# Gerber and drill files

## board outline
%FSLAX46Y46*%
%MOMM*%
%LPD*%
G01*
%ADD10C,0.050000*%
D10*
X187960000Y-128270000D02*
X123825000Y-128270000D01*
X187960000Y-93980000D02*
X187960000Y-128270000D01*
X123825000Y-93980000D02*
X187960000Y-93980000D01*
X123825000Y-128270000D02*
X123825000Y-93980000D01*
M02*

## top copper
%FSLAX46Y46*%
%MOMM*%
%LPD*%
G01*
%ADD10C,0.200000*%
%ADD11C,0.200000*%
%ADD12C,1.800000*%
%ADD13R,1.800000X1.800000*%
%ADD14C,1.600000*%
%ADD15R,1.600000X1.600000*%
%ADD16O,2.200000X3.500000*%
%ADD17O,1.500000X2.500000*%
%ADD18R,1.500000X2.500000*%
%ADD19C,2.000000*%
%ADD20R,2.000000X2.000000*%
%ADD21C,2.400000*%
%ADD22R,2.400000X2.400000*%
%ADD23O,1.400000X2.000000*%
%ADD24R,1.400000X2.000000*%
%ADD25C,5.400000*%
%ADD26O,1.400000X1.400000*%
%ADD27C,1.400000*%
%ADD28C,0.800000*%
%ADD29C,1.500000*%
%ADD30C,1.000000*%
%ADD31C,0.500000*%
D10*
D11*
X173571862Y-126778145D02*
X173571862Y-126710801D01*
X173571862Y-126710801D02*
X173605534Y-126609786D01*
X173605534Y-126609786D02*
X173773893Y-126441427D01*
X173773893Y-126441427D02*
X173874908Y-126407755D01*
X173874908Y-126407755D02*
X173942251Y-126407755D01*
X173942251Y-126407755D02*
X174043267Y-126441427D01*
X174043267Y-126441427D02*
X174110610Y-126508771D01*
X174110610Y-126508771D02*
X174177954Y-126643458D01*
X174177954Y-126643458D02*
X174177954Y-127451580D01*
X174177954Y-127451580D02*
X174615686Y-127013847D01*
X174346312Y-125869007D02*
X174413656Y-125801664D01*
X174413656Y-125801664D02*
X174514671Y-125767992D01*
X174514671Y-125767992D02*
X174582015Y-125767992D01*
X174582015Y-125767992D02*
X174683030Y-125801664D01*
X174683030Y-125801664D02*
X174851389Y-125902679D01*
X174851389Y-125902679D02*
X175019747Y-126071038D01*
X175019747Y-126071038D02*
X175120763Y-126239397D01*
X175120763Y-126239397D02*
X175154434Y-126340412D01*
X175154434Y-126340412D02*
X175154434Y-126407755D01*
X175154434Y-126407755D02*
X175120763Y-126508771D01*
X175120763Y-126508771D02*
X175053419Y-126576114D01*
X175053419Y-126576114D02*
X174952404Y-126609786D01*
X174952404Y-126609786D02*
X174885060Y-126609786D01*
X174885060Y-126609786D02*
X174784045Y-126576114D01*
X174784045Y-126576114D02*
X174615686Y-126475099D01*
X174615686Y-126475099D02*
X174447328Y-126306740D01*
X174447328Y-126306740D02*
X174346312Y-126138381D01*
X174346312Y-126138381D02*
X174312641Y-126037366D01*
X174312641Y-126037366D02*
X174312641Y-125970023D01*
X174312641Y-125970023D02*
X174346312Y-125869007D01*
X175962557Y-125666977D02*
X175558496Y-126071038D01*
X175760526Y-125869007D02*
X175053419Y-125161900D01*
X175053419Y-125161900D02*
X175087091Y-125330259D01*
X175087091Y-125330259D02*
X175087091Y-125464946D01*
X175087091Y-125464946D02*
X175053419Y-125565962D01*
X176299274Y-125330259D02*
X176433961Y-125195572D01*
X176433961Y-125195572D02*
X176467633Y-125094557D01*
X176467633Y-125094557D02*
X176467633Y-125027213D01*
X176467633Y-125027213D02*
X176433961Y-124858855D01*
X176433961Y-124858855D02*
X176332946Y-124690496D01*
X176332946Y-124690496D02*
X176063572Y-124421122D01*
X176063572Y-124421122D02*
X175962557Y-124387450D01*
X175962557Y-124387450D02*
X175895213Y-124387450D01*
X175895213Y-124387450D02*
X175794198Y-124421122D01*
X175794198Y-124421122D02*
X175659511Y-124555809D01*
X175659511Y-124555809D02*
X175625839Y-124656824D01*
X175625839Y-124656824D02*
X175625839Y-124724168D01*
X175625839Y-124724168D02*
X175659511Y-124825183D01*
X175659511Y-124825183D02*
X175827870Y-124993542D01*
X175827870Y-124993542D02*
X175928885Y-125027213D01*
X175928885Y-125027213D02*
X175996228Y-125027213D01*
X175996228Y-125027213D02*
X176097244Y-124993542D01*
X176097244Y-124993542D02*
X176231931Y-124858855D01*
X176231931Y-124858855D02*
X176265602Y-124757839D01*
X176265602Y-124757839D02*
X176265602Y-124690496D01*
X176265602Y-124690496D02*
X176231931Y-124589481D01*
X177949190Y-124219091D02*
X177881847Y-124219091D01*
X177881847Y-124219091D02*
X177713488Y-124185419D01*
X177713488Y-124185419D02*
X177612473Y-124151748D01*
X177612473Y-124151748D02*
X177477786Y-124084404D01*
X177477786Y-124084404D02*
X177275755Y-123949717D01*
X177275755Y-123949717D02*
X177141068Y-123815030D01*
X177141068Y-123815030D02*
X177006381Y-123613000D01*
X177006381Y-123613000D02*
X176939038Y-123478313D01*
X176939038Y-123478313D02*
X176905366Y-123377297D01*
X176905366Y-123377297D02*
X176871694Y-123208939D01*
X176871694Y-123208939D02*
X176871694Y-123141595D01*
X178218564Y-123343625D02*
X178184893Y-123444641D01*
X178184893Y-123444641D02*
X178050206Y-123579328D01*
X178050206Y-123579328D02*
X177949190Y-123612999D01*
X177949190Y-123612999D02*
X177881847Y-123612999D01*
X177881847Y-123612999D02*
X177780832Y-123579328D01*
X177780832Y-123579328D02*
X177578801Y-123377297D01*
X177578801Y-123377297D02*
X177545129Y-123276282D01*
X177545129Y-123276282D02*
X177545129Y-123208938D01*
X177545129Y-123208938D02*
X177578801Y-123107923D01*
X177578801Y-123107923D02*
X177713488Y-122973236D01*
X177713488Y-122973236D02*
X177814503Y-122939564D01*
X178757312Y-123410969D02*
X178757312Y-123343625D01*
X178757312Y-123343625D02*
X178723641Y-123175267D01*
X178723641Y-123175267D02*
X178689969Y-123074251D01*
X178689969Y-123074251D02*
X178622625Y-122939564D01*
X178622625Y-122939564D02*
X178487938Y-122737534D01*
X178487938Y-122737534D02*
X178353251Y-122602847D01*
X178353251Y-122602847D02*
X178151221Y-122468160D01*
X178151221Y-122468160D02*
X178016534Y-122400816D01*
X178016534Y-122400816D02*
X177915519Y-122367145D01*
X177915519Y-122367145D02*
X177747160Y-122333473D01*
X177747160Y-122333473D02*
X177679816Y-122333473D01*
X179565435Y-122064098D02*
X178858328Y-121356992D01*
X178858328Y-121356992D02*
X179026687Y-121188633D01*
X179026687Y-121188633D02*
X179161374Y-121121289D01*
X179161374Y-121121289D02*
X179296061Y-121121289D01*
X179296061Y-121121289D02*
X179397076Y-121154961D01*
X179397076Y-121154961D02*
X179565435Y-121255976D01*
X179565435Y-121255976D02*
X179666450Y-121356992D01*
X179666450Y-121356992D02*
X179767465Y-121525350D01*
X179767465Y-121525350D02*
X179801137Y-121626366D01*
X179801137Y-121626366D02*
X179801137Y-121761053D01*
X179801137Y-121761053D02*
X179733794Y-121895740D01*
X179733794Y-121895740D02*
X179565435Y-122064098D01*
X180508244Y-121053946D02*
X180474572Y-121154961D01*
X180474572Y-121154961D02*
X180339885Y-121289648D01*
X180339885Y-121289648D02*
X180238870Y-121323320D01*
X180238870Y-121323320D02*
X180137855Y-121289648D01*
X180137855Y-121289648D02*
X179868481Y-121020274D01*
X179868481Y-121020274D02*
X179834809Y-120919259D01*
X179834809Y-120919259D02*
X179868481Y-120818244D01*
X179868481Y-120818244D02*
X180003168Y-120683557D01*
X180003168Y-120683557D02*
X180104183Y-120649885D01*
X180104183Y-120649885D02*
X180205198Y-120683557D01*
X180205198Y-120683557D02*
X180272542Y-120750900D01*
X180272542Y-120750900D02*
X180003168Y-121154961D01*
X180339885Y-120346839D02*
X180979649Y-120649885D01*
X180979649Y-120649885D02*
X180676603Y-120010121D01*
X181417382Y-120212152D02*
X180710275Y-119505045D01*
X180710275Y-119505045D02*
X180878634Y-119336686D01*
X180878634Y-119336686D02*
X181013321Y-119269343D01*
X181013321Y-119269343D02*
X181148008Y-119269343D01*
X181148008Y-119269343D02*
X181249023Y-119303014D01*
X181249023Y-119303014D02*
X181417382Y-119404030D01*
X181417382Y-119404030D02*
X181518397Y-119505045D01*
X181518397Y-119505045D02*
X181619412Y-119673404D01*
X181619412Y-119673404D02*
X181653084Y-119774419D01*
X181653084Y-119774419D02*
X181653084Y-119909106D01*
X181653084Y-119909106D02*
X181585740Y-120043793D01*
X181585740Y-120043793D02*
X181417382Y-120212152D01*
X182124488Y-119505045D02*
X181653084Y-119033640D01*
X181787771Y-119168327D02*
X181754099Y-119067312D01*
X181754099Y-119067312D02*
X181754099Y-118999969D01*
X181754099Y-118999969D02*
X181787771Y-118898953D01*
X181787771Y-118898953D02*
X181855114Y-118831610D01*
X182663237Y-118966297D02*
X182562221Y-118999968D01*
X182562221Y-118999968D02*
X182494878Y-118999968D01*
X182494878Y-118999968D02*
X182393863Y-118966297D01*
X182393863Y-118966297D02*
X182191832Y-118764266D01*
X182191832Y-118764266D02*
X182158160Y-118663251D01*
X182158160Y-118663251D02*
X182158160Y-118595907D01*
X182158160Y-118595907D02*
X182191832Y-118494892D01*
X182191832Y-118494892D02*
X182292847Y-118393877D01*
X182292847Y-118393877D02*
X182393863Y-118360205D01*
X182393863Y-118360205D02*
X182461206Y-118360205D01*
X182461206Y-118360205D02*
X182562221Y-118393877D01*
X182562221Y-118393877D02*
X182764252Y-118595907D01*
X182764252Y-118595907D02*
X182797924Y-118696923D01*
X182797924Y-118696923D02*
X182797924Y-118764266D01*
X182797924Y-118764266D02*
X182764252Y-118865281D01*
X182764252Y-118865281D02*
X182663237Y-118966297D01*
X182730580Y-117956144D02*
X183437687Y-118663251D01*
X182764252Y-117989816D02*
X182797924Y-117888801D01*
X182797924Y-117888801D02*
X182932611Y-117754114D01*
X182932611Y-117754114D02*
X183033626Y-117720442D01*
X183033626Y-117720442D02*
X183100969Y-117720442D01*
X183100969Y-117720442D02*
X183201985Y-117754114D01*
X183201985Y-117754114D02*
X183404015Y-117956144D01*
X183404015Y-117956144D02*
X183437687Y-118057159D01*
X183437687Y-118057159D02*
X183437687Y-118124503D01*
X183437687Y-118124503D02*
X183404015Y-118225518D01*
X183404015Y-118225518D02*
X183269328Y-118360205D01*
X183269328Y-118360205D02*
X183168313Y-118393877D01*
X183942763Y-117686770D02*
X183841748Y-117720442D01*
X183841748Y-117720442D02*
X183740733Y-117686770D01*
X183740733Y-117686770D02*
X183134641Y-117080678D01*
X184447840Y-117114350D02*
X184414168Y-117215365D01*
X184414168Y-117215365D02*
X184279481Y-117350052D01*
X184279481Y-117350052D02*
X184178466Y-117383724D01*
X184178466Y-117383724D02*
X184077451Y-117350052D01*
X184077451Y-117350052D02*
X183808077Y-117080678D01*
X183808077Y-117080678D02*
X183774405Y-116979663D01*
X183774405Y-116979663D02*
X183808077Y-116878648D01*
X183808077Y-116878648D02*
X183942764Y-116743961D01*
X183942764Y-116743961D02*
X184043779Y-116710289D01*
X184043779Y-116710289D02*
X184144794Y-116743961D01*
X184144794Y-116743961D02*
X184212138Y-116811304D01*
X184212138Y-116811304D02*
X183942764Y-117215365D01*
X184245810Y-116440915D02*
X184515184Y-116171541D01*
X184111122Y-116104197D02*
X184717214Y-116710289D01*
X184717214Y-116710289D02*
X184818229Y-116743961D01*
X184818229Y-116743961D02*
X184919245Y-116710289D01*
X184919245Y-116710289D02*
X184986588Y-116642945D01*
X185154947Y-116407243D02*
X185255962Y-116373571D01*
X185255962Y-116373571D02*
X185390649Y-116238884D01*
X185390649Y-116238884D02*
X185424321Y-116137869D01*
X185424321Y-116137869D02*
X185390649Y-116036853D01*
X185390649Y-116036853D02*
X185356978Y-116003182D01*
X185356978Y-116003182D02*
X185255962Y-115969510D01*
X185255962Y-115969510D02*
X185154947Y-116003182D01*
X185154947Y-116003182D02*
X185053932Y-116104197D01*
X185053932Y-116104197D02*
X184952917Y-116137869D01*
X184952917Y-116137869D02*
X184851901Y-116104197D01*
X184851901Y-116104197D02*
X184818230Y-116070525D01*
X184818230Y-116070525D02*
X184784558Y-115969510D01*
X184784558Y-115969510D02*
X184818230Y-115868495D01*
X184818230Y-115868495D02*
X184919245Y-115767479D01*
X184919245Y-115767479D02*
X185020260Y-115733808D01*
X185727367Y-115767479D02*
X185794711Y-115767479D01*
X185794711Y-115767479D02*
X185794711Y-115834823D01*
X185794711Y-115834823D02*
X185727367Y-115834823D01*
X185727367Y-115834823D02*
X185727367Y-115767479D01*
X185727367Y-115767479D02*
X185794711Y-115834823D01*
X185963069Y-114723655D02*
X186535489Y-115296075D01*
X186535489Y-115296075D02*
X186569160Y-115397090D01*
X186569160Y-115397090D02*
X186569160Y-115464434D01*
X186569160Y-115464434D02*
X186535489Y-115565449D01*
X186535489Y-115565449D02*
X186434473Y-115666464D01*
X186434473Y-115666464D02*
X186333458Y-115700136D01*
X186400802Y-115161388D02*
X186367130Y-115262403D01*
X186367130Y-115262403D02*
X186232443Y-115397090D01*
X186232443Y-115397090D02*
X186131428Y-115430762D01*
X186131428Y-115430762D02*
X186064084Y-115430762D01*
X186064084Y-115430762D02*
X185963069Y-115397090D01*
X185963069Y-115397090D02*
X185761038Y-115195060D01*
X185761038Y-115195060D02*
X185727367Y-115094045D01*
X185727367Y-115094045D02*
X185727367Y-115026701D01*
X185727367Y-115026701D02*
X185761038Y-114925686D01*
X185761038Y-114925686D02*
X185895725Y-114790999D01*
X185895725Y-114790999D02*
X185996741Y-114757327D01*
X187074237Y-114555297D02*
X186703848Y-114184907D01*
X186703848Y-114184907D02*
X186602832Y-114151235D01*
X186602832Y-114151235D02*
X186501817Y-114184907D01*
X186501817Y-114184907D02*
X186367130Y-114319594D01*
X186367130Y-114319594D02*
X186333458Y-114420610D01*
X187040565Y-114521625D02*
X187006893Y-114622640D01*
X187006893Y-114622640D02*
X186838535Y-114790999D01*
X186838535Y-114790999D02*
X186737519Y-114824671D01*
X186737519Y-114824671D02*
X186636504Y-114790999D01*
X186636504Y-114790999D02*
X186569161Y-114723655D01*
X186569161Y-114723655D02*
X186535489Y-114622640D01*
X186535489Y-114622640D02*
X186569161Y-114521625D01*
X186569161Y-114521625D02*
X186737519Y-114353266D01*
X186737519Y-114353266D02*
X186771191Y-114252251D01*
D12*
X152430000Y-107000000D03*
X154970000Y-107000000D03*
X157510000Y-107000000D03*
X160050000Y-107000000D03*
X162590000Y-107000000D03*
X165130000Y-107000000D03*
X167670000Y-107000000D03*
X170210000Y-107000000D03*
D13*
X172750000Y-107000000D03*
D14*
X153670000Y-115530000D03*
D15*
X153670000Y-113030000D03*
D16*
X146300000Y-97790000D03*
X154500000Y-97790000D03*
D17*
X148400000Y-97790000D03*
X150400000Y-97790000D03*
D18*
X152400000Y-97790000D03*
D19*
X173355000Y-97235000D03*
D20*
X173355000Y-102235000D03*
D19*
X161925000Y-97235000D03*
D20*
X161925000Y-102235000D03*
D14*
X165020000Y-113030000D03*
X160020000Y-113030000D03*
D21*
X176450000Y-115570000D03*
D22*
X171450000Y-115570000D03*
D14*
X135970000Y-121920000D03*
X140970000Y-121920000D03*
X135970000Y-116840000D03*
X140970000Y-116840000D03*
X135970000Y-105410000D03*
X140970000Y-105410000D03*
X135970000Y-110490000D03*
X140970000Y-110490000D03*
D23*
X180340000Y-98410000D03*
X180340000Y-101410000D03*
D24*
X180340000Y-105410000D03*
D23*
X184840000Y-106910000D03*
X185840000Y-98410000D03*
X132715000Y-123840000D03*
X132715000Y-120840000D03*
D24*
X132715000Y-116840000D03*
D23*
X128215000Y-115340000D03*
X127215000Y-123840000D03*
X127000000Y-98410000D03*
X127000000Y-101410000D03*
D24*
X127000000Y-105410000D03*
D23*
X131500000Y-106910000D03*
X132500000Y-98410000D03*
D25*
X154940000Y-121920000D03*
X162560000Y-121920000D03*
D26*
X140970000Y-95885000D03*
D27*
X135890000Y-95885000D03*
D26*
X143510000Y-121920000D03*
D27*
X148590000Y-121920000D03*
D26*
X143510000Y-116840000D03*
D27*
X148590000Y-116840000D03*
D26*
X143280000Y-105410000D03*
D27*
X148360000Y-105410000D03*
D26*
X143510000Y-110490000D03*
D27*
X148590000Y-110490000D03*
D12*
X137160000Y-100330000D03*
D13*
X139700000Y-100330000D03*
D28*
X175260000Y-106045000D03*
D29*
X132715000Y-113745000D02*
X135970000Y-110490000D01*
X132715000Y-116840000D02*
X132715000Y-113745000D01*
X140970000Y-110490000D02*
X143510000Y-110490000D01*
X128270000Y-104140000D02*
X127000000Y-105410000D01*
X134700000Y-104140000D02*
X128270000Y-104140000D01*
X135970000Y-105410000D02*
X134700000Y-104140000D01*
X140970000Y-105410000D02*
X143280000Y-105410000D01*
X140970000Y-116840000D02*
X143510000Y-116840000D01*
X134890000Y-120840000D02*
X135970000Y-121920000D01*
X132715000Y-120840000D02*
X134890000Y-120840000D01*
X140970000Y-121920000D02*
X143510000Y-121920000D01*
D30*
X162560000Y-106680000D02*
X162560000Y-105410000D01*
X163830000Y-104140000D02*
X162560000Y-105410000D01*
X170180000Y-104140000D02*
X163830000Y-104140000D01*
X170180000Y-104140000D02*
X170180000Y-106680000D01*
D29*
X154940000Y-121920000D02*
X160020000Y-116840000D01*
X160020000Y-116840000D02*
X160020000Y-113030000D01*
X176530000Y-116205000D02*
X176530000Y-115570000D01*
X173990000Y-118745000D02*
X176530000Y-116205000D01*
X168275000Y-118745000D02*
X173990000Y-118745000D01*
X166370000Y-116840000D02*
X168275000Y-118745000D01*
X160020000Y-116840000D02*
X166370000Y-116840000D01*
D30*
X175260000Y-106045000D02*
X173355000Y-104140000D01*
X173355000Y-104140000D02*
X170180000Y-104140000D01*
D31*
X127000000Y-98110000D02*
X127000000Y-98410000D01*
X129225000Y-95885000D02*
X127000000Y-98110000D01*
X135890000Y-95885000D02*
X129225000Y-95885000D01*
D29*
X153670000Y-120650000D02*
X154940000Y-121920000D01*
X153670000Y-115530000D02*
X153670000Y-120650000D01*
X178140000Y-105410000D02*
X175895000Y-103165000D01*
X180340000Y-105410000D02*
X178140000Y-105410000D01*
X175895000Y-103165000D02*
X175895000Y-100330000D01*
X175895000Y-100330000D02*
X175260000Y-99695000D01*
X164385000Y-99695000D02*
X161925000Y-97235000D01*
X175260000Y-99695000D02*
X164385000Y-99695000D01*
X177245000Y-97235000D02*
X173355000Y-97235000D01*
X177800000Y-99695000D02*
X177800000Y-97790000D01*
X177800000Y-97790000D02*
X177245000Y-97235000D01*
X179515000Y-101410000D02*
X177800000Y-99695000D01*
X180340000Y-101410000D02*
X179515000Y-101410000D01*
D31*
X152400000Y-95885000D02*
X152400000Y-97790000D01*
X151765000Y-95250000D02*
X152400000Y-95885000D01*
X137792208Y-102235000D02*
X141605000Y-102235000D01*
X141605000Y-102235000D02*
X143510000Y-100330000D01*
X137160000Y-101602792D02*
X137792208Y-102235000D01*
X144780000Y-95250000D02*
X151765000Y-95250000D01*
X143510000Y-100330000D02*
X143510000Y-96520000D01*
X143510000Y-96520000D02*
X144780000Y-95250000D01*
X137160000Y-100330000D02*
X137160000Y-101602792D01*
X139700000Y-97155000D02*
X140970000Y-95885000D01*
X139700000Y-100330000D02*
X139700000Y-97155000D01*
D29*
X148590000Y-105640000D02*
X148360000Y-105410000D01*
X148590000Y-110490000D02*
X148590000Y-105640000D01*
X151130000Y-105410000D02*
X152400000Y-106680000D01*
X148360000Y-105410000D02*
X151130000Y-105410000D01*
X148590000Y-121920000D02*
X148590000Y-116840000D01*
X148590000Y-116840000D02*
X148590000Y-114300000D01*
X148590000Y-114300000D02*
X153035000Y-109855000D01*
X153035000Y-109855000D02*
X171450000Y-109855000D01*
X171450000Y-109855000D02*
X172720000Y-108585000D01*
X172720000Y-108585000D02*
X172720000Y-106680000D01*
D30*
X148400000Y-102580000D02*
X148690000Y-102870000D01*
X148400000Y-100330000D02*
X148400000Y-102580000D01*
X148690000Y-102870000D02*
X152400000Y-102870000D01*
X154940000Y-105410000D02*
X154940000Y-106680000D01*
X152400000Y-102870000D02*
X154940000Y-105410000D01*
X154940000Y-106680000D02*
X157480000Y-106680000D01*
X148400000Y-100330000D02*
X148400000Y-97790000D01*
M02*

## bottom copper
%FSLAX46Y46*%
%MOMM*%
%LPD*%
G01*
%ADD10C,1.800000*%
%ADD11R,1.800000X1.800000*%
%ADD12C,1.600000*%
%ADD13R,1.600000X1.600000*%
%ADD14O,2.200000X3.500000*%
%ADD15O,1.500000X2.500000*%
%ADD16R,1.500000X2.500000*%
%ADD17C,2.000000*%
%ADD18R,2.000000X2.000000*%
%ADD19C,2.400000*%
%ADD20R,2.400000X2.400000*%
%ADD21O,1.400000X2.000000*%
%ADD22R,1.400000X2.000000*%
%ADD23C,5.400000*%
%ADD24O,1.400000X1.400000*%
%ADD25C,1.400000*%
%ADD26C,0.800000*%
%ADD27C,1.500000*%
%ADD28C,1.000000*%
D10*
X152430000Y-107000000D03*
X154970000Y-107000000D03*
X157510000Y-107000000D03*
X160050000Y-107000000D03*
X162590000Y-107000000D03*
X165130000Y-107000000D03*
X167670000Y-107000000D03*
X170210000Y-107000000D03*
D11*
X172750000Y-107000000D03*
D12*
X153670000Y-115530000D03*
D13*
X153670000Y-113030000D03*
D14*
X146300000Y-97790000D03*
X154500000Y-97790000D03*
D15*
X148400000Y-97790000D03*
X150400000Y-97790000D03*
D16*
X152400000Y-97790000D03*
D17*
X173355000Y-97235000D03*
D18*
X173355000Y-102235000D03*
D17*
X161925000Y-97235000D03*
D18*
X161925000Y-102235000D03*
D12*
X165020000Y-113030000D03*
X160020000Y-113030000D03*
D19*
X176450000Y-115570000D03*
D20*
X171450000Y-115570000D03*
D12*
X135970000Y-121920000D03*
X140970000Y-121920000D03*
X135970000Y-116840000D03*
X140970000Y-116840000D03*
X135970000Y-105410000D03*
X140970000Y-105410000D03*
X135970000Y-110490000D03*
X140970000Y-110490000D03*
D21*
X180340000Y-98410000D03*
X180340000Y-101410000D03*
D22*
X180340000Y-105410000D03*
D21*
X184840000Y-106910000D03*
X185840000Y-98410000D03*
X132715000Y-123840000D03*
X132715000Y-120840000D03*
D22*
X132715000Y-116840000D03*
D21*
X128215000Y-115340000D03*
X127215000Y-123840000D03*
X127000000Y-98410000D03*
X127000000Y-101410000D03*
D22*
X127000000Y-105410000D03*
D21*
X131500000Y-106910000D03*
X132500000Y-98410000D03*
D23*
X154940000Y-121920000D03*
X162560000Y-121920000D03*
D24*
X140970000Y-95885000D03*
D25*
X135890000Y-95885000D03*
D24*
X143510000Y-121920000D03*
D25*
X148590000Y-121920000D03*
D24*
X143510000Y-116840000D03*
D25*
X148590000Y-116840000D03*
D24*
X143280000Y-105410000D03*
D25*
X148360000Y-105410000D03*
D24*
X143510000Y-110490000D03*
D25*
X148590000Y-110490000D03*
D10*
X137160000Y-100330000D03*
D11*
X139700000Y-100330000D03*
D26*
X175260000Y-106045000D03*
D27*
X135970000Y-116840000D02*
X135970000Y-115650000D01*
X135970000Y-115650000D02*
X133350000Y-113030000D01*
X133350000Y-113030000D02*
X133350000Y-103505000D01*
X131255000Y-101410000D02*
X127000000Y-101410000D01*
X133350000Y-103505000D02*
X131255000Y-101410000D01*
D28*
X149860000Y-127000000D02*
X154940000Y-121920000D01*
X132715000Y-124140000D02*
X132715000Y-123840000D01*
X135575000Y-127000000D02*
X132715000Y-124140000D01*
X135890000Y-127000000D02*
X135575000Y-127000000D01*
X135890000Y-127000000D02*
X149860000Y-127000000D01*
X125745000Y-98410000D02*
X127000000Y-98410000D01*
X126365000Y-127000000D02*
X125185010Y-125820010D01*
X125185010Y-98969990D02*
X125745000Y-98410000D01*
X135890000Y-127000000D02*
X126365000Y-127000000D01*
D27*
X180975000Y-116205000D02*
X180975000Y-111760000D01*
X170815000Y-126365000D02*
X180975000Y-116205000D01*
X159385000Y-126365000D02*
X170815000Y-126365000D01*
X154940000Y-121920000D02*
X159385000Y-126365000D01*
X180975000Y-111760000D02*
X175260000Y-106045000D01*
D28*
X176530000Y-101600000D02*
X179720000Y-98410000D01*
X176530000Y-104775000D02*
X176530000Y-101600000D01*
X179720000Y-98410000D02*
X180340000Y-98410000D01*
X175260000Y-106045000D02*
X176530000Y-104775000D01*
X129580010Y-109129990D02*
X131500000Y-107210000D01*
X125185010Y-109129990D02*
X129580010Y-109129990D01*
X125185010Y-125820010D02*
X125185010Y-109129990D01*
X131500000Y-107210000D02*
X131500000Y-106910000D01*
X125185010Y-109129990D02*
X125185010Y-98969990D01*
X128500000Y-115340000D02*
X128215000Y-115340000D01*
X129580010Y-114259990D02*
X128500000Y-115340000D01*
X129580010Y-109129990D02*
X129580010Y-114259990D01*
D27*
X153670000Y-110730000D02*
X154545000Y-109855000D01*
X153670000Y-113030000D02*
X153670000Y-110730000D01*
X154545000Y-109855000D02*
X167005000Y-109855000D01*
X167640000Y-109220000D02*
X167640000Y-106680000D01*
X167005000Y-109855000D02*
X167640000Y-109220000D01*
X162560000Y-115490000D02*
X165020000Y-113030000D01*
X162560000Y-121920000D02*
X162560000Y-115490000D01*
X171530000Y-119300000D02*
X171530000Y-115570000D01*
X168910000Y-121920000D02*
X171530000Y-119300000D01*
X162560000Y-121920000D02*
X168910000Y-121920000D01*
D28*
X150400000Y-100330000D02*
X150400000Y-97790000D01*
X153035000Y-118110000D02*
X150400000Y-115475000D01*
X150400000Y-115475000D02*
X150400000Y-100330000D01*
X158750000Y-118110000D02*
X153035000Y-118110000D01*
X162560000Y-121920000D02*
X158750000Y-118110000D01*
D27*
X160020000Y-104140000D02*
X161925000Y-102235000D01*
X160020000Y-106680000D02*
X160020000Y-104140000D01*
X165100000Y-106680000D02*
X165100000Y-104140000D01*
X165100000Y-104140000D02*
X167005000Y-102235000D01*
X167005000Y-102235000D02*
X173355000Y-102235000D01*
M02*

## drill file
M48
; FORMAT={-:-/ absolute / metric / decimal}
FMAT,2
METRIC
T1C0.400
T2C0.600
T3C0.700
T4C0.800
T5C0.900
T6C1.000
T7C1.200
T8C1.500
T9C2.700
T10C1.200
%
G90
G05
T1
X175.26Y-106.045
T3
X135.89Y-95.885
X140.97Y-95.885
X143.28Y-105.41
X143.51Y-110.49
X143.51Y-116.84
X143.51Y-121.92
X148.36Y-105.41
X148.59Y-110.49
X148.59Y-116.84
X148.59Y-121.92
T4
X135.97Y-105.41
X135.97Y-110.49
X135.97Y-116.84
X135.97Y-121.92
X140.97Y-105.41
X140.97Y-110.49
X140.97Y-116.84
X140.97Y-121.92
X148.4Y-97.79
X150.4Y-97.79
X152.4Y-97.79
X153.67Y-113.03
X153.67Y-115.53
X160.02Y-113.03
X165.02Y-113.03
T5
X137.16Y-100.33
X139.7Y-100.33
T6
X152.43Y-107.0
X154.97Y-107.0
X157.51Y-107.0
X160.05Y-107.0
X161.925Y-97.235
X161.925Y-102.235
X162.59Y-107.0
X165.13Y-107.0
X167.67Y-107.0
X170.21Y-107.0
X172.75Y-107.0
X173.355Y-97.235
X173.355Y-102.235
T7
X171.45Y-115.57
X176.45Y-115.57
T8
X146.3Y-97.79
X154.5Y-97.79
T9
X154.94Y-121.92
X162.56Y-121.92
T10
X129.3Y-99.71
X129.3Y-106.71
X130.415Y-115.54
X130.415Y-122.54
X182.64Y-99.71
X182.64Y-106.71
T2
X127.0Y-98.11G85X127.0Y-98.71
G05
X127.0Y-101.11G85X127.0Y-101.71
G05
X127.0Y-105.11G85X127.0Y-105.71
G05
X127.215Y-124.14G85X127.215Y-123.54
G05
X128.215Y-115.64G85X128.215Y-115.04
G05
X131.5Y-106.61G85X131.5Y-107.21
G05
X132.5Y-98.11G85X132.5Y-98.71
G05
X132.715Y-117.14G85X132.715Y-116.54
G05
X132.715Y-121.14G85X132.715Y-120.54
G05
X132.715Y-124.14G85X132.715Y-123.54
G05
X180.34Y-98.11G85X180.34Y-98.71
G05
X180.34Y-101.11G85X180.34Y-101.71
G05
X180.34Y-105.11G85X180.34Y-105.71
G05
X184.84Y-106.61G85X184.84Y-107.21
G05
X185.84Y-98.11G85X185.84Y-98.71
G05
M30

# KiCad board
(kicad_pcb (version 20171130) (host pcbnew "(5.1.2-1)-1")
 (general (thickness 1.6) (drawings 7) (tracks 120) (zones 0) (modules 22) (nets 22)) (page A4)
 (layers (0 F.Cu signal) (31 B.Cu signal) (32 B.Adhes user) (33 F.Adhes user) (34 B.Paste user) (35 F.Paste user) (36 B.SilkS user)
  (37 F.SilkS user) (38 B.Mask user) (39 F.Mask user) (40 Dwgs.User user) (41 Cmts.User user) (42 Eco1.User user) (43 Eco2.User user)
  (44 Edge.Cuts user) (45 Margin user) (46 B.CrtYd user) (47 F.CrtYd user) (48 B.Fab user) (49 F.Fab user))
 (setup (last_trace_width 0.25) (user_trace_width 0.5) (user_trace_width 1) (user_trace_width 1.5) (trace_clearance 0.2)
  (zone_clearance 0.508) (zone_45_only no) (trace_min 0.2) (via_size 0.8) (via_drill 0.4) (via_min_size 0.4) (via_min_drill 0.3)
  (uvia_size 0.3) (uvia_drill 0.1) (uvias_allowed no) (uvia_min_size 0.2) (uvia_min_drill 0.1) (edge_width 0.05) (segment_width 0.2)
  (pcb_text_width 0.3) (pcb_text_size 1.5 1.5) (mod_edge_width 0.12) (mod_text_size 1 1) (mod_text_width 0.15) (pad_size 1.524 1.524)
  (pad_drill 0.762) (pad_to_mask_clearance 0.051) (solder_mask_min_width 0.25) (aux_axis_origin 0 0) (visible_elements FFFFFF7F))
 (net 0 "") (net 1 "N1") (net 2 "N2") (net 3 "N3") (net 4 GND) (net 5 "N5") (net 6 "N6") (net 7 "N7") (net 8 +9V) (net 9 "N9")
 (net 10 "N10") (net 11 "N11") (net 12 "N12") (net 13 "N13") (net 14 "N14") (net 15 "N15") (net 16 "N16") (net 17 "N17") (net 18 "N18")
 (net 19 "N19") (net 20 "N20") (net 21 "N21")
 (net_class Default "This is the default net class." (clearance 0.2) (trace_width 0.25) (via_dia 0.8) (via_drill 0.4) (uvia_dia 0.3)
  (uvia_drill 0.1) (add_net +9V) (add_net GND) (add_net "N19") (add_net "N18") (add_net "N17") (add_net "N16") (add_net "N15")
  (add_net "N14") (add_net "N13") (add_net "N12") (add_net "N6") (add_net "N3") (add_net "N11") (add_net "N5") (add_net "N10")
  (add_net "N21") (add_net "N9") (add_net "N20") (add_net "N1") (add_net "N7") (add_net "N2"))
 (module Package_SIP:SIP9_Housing (layer F.Cu) (at 172.75 107 180)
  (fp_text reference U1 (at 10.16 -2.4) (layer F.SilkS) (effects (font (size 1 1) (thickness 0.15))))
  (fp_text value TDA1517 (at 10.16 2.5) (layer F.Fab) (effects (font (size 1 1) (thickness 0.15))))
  (pad 9 thru_hole circle (at 20.32 0 270) (size 1.8 1.8) (drill 1) (layers *.Cu *.Mask) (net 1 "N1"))
  (pad 8 thru_hole circle (at 17.78 0 270) (size 1.8 1.8) (drill 1) (layers *.Cu *.Mask) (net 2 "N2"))
  (pad 7 thru_hole circle (at 15.24 0 270) (size 1.8 1.8) (drill 1) (layers *.Cu *.Mask) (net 2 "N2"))
  (pad 6 thru_hole circle (at 12.7 0 270) (size 1.8 1.8) (drill 1) (layers *.Cu *.Mask) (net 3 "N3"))
  (pad 5 thru_hole circle (at 10.16 0 270) (size 1.8 1.8) (drill 1) (layers *.Cu *.Mask) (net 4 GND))
  (pad 4 thru_hole circle (at 7.62 0 270) (size 1.8 1.8) (drill 1) (layers *.Cu *.Mask) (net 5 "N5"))
  (pad 3 thru_hole circle (at 5.08 0 270) (size 1.8 1.8) (drill 1) (layers *.Cu *.Mask) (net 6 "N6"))
  (pad 2 thru_hole circle (at 2.54 0 270) (size 1.8 1.8) (drill 1) (layers *.Cu *.Mask) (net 4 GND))
  (pad 1 thru_hole rect (at 0 0 270) (size 1.8 1.8) (drill 1) (layers *.Cu *.Mask) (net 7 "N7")))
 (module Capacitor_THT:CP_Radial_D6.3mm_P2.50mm (layer F.Cu) (at 153.67 113.03 270)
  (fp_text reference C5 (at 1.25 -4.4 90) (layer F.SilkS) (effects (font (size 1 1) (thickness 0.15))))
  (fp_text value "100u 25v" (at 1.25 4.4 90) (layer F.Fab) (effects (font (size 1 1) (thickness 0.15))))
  (pad 2 thru_hole circle (at 2.5 0 270) (size 1.6 1.6) (drill 0.8) (layers *.Cu *.Mask) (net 4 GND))
  (pad 1 thru_hole rect (at 0 0 270) (size 1.6 1.6) (drill 0.8) (layers *.Cu *.Mask) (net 6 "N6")))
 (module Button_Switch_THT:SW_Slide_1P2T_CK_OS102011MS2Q (layer F.Cu) (at 152.4 97.79 180)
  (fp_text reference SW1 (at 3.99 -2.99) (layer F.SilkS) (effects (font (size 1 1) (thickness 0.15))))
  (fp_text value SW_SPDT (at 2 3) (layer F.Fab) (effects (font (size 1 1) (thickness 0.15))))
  (pad "" thru_hole oval (at 6.1 0 180) (size 2.2 3.5) (drill 1.5) (layers *.Cu *.Mask))
  (pad "" thru_hole oval (at -2.1 0 180) (size 2.2 3.5) (drill 1.5) (layers *.Cu *.Mask))
  (pad 3 thru_hole oval (at 4 0 180) (size 1.5 2.5) (drill 0.8) (layers *.Cu *.Mask) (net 2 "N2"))
  (pad 2 thru_hole oval (at 2 0 180) (size 1.5 2.5) (drill 0.8) (layers *.Cu *.Mask) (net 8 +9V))
  (pad 1 thru_hole rect (at 0 0 180) (size 1.5 2.5) (drill 0.8) (layers *.Cu *.Mask) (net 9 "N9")))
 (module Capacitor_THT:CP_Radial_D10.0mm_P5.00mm (layer F.Cu) (at 173.355 102.235 90)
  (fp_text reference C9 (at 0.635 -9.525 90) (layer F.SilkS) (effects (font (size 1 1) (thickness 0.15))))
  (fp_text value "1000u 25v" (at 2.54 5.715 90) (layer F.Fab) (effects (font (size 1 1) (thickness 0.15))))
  (pad 2 thru_hole circle (at 5 0 90) (size 2 2) (drill 1) (layers *.Cu *.Mask) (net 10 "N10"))
  (pad 1 thru_hole rect (at 0 0 90) (size 2 2) (drill 1) (layers *.Cu *.Mask) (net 5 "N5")))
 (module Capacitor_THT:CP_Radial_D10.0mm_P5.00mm (layer F.Cu) (at 161.925 102.235 90)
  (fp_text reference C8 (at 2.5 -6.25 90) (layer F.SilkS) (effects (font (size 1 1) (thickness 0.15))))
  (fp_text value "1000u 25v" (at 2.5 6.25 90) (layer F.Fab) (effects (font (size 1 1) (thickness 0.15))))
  (pad 2 thru_hole circle (at 5 0 90) (size 2 2) (drill 1) (layers *.Cu *.Mask) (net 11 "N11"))
  (pad 1 thru_hole rect (at 0 0 90) (size 2 2) (drill 1) (layers *.Cu *.Mask) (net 3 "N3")))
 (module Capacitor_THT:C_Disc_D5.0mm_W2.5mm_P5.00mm (layer F.Cu) (at 160.02 113.03)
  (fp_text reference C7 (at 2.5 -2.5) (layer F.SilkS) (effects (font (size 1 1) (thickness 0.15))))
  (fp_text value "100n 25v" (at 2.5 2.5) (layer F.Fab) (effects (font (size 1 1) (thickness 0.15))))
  (pad 2 thru_hole circle (at 5 0) (size 1.6 1.6) (drill 0.8) (layers *.Cu *.Mask) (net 8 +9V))
  (pad 1 thru_hole circle (at 0 0) (size 1.6 1.6) (drill 0.8) (layers *.Cu *.Mask) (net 4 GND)))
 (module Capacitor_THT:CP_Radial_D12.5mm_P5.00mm (layer F.Cu) (at 171.45 115.57)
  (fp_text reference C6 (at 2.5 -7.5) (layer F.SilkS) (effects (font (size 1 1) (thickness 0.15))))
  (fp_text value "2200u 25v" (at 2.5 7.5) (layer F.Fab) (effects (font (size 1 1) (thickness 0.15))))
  (pad 2 thru_hole circle (at 5 0) (size 2.4 2.4) (drill 1.2) (layers *.Cu *.Mask) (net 4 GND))
  (pad 1 thru_hole rect (at 0 0) (size 2.4 2.4) (drill 1.2) (layers *.Cu *.Mask) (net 8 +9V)))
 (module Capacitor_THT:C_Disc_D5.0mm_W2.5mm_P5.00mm (layer F.Cu) (at 140.97 121.92 180)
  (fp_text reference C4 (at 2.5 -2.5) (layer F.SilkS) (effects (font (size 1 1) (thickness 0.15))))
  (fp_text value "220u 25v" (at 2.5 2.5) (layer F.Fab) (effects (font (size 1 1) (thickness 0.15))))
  (pad 2 thru_hole circle (at 5 0 180) (size 1.6 1.6) (drill 0.8) (layers *.Cu *.Mask) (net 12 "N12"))
  (pad 1 thru_hole circle (at 0 0 180) (size 1.6 1.6) (drill 0.8) (layers *.Cu *.Mask) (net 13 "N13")))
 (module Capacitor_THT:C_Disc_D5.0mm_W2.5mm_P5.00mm (layer F.Cu) (at 140.97 116.84 180)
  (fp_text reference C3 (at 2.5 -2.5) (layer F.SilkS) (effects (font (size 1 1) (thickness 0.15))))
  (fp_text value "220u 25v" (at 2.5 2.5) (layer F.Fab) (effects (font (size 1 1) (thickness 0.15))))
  (pad 2 thru_hole circle (at 5 0 180) (size 1.6 1.6) (drill 0.8) (layers *.Cu *.Mask) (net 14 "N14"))
  (pad 1 thru_hole circle (at 0 0 180) (size 1.6 1.6) (drill 0.8) (layers *.Cu *.Mask) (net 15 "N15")))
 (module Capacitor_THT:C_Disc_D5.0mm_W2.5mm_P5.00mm (layer F.Cu) (at 140.97 105.41 180)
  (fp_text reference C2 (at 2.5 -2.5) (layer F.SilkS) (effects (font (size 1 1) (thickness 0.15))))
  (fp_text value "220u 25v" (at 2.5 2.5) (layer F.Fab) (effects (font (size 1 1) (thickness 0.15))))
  (pad 2 thru_hole circle (at 5 0 180) (size 1.6 1.6) (drill 0.8) (layers *.Cu *.Mask) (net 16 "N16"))
  (pad 1 thru_hole circle (at 0 0 180) (size 1.6 1.6) (drill 0.8) (layers *.Cu *.Mask) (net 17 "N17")))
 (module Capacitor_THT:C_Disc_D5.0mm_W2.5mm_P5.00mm (layer F.Cu) (at 140.97 110.49 180)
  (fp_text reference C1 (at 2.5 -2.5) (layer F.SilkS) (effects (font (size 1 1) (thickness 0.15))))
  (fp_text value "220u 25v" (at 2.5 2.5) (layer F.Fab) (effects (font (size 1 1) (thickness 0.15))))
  (pad 2 thru_hole circle (at 5 0 180) (size 1.6 1.6) (drill 0.8) (layers *.Cu *.Mask) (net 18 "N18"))
  (pad 1 thru_hole circle (at 0 0 180) (size 1.6 1.6) (drill 0.8) (layers *.Cu *.Mask) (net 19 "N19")))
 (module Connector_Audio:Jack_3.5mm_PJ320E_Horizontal (layer F.Cu) (at 180.34 105.41)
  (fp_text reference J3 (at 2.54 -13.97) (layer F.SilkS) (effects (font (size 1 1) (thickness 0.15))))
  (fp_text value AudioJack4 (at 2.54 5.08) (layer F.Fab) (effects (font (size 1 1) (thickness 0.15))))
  (pad "" np_thru_hole circle (at 2.3 1.3 270) (size 1.2 1.2) (drill 1.2) (layers *.Cu *.Mask))
  (pad "" np_thru_hole circle (at 2.3 -5.7 270) (size 1.2 1.2) (drill 1.2) (layers *.Cu *.Mask))
  (pad R2 thru_hole oval (at 0 -7 270) (size 2 1.4) (drill oval 1.2 0.6) (layers *.Cu *.Mask) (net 4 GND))
  (pad R1 thru_hole oval (at 0 -4 270) (size 2 1.4) (drill oval 1.2 0.6) (layers *.Cu *.Mask) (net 10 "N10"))
  (pad T thru_hole rect (at 0 0 270) (size 2 1.4) (drill oval 1.2 0.6) (layers *.Cu *.Mask) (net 11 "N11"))
  (pad S thru_hole oval (at 4.5 1.5 270) (size 2 1.4) (drill oval 1.2 0.6) (layers *.Cu *.Mask) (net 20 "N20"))
  (pad "" thru_hole oval (at 5.5 -7 270) (size 2 1.4) (drill oval 1.2 0.6) (layers *.Cu *.Mask)))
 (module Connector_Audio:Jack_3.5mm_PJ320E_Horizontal (layer F.Cu) (at 132.715 116.84 180)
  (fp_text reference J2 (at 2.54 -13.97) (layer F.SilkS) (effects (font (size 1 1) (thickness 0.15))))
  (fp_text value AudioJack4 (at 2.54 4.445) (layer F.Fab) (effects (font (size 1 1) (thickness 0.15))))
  (pad "" np_thru_hole circle (at 2.3 1.3 90) (size 1.2 1.2) (drill 1.2) (layers *.Cu *.Mask))
  (pad "" np_thru_hole circle (at 2.3 -5.7 90) (size 1.2 1.2) (drill 1.2) (layers *.Cu *.Mask))
  (pad R2 thru_hole oval (at 0 -7 90) (size 2 1.4) (drill oval 1.2 0.6) (layers *.Cu *.Mask) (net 4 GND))
  (pad R1 thru_hole oval (at 0 -4 90) (size 2 1.4) (drill oval 1.2 0.6) (layers *.Cu *.Mask) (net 12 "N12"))
  (pad T thru_hole rect (at 0 0 90) (size 2 1.4) (drill oval 1.2 0.6) (layers *.Cu *.Mask) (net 18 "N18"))
  (pad S thru_hole oval (at 4.5 1.5 90) (size 2 1.4) (drill oval 1.2 0.6) (layers *.Cu *.Mask) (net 4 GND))
  (pad "" thru_hole oval (at 5.5 -7 90) (size 2 1.4) (drill oval 1.2 0.6) (layers *.Cu *.Mask)))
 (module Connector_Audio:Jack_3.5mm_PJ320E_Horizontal (layer F.Cu) (at 127 105.41)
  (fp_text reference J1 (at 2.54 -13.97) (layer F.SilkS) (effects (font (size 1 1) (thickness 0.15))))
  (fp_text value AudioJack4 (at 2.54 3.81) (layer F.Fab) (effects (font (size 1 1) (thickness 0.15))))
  (pad "" np_thru_hole circle (at 2.3 1.3 270) (size 1.2 1.2) (drill 1.2) (layers *.Cu *.Mask))
  (pad "" np_thru_hole circle (at 2.3 -5.7 270) (size 1.2 1.2) (drill 1.2) (layers *.Cu *.Mask))
  (pad R2 thru_hole oval (at 0 -7 270) (size 2 1.4) (drill oval 1.2 0.6) (layers *.Cu *.Mask) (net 4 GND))
  (pad R1 thru_hole oval (at 0 -4 270) (size 2 1.4) (drill oval 1.2 0.6) (layers *.Cu *.Mask) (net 14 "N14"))
  (pad T thru_hole rect (at 0 0 270) (size 2 1.4) (drill oval 1.2 0.6) (layers *.Cu *.Mask) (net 16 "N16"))
  (pad S thru_hole oval (at 4.5 1.5 270) (size 2 1.4) (drill oval 1.2 0.6) (layers *.Cu *.Mask) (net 4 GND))
  (pad "" thru_hole oval (at 5.5 -7 270) (size 2 1.4) (drill oval 1.2 0.6) (layers *.Cu *.Mask)))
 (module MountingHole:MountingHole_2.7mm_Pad (layer F.Cu) (at 154.94 121.92)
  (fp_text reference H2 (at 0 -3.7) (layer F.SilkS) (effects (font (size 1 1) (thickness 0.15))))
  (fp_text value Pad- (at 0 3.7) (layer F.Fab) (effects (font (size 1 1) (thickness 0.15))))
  (pad 1 thru_hole circle (at 0 0) (size 5.4 5.4) (drill 2.7) (layers *.Cu *.Mask) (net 4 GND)))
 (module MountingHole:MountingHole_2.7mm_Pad (layer F.Cu) (at 162.56 121.92)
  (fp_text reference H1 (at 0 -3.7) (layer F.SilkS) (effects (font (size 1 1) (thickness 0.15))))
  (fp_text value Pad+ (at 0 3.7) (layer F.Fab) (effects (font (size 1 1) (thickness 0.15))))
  (pad 1 thru_hole circle (at 0 0) (size 5.4 5.4) (drill 2.7) (layers *.Cu *.Mask) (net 8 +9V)))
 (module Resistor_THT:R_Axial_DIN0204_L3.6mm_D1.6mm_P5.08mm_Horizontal (layer F.Cu) (at 135.89 95.885)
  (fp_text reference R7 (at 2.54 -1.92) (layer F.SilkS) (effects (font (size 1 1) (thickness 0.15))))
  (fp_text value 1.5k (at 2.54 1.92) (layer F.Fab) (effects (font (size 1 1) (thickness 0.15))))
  (pad 2 thru_hole oval (at 5.08 0) (size 1.4 1.4) (drill 0.7) (layers *.Cu *.Mask) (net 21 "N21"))
  (pad 1 thru_hole circle (at 0 0) (size 1.4 1.4) (drill 0.7) (layers *.Cu *.Mask) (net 4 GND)))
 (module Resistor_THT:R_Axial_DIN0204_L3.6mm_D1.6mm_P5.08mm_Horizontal (layer F.Cu) (at 148.59 121.92 180)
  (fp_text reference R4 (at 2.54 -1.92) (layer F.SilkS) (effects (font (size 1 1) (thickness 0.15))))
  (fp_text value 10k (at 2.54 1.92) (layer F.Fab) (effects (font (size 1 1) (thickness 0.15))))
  (pad 2 thru_hole oval (at 5.08 0 180) (size 1.4 1.4) (drill 0.7) (layers *.Cu *.Mask) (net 13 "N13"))
  (pad 1 thru_hole circle (at 0 0 180) (size 1.4 1.4) (drill 0.7) (layers *.Cu *.Mask) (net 7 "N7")))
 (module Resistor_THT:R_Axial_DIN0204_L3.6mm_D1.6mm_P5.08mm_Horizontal (layer F.Cu) (at 148.59 116.84 180)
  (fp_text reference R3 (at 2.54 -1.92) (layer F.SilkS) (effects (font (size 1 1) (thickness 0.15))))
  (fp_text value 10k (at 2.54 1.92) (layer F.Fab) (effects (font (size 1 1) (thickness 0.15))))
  (pad 2 thru_hole oval (at 5.08 0 180) (size 1.4 1.4) (drill 0.7) (layers *.Cu *.Mask) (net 15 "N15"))
  (pad 1 thru_hole circle (at 0 0 180) (size 1.4 1.4) (drill 0.7) (layers *.Cu *.Mask) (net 7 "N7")))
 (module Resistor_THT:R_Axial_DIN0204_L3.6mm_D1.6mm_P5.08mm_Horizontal (layer F.Cu) (at 148.36 105.41 180)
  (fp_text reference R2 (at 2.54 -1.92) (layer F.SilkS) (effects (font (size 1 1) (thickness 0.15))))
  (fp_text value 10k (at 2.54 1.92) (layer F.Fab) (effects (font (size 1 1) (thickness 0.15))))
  (pad 2 thru_hole oval (at 5.08 0 180) (size 1.4 1.4) (drill 0.7) (layers *.Cu *.Mask) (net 17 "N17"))
  (pad 1 thru_hole circle (at 0 0 180) (size 1.4 1.4) (drill 0.7) (layers *.Cu *.Mask) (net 1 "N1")))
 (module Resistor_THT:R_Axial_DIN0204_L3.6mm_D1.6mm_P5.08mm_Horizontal (layer F.Cu) (at 148.59 110.49 180)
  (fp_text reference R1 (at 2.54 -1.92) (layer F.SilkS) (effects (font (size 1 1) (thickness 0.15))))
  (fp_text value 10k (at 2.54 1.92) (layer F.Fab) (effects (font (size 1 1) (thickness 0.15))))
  (pad 2 thru_hole oval (at 5.08 0 180) (size 1.4 1.4) (drill 0.7) (layers *.Cu *.Mask) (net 19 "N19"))
  (pad 1 thru_hole circle (at 0 0 180) (size 1.4 1.4) (drill 0.7) (layers *.Cu *.Mask) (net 1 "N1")))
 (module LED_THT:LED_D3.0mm (layer F.Cu) (at 139.7 100.33 180)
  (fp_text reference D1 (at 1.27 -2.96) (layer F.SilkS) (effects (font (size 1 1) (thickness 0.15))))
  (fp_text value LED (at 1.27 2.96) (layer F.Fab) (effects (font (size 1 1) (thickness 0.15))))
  (pad 2 thru_hole circle (at 2.54 0 180) (size 1.8 1.8) (drill 0.9) (layers *.Cu *.Mask) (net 9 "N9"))
  (pad 1 thru_hole rect (at 0 0 180) (size 1.8 1.8) (drill 0.9) (layers *.Cu *.Mask) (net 21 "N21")))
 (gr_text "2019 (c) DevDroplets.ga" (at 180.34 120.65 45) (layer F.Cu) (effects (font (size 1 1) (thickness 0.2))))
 (gr_line (start 187.96 128.27) (end 123.825 128.27) (layer Edge.Cuts) (width 0.05))
 (gr_line (start 187.96 93.98) (end 187.96 128.27) (layer Edge.Cuts) (width 0.05))
 (gr_line (start 123.825 93.98) (end 187.96 93.98) (layer Edge.Cuts) (width 0.05))
 (gr_line (start 123.825 128.27) (end 123.825 93.98) (layer Edge.Cuts) (width 0.05))
 (segment (start 132.715 113.745) (end 135.97 110.49) (width 1.5) (layer F.Cu) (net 18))
 (segment (start 132.715 116.84) (end 132.715 113.745) (width 1.5) (layer F.Cu) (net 18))
 (segment (start 140.97 110.49) (end 143.51 110.49) (width 1.5) (layer F.Cu) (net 19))
 (segment (start 128.27 104.14) (end 127 105.41) (width 1.5) (layer F.Cu) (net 16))
 (segment (start 134.7 104.14) (end 128.27 104.14) (width 1.5) (layer F.Cu) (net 16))
 (segment (start 135.97 105.41) (end 134.7 104.14) (width 1.5) (layer F.Cu) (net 16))
 (segment (start 140.97 105.41) (end 143.28 105.41) (width 1.5) (layer F.Cu) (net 17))
 (segment (start 135.97 116.84) (end 135.97 115.65) (width 1.5) (layer B.Cu) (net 14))
 (segment (start 135.97 115.65) (end 133.35 113.03) (width 1.5) (layer B.Cu) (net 14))
 (segment (start 133.35 113.03) (end 133.35 103.505) (width 1.5) (layer B.Cu) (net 14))
 (segment (start 131.255 101.41) (end 127 101.41) (width 1.5) (layer B.Cu) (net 14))
 (segment (start 133.35 103.505) (end 131.255 101.41) (width 1.5) (layer B.Cu) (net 14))
 (segment (start 140.97 116.84) (end 143.51 116.84) (width 1.5) (layer F.Cu) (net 15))
 (segment (start 134.89 120.84) (end 135.97 121.92) (width 1.5) (layer F.Cu) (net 12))
 (segment (start 132.715 120.84) (end 134.89 120.84) (width 1.5) (layer F.Cu) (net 12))
 (segment (start 140.97 121.92) (end 143.51 121.92) (width 1.5) (layer F.Cu) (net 13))
 (segment (start 149.86 127) (end 154.94 121.92) (width 1) (layer B.Cu) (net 4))
 (segment (start 132.715 124.14) (end 132.715 123.84) (width 1) (layer B.Cu) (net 4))
 (segment (start 135.575 127) (end 132.715 124.14) (width 1) (layer B.Cu) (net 4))
 (segment (start 135.89 127) (end 135.575 127) (width 1) (layer B.Cu) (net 4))
 (segment (start 135.89 127) (end 149.86 127) (width 1) (layer B.Cu) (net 4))
 (segment (start 162.56 106.68) (end 162.56 105.41) (width 1) (layer F.Cu) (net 4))
 (segment (start 163.83 104.14) (end 162.56 105.41) (width 1) (layer F.Cu) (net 4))
 (segment (start 170.18 104.14) (end 163.83 104.14) (width 1) (layer F.Cu) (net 4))
 (segment (start 170.18 104.14) (end 170.18 106.68) (width 1) (layer F.Cu) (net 4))
 (segment (start 125.745 98.41) (end 127 98.41) (width 1) (layer B.Cu) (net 4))
 (segment (start 126.365 127) (end 125.18501 125.82001) (width 1) (layer B.Cu) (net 4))
 (segment (start 125.18501 98.96999) (end 125.745 98.41) (width 1) (layer B.Cu) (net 4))
 (segment (start 135.89 127) (end 126.365 127) (width 1) (layer B.Cu) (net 4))
 (segment (start 180.975 116.205) (end 180.975 111.76) (width 1.5) (layer B.Cu) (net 4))
 (segment (start 170.815 126.365) (end 180.975 116.205) (width 1.5) (layer B.Cu) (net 4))
 (segment (start 159.385 126.365) (end 170.815 126.365) (width 1.5) (layer B.Cu) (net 4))
 (segment (start 154.94 121.92) (end 159.385 126.365) (width 1.5) (layer B.Cu) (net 4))
 (segment (start 154.94 121.92) (end 160.02 116.84) (width 1.5) (layer F.Cu) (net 4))
 (segment (start 160.02 116.84) (end 160.02 113.03) (width 1.5) (layer F.Cu) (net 4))
 (segment (start 176.53 116.205) (end 176.53 115.57) (width 1.5) (layer F.Cu) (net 4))
 (segment (start 173.99 118.745) (end 176.53 116.205) (width 1.5) (layer F.Cu) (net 4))
 (segment (start 168.275 118.745) (end 173.99 118.745) (width 1.5) (layer F.Cu) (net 4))
 (segment (start 166.37 116.84) (end 168.275 118.745) (width 1.5) (layer F.Cu) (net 4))
 (segment (start 160.02 116.84) (end 166.37 116.84) (width 1.5) (layer F.Cu) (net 4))
 (via (at 175.26 106.045) (size 0.8) (drill 0.4) (layers F.Cu B.Cu) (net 4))
 (segment (start 180.975 111.76) (end 175.26 106.045) (width 1.5) (layer B.Cu) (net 4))
 (segment (start 175.26 106.045) (end 173.355 104.14) (width 1) (layer F.Cu) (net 4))
 (segment (start 173.355 104.14) (end 170.18 104.14) (width 1) (layer F.Cu) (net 4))
 (segment (start 176.53 101.6) (end 179.72 98.41) (width 1) (layer B.Cu) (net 4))
 (segment (start 176.53 104.775) (end 176.53 101.6) (width 1) (layer B.Cu) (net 4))
 (segment (start 179.72 98.41) (end 180.34 98.41) (width 1) (layer B.Cu) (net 4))
 (segment (start 175.26 106.045) (end 176.53 104.775) (width 1) (layer B.Cu) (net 4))
 (segment (start 127 98.11) (end 127 98.41) (width 0.5) (layer F.Cu) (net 4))
 (segment (start 129.225 95.885) (end 127 98.11) (width 0.5) (layer F.Cu) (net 4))
 (segment (start 135.89 95.885) (end 129.225 95.885) (width 0.5) (layer F.Cu) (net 4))
 (segment (start 153.67 120.65) (end 154.94 121.92) (width 1.5) (layer F.Cu) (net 4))
 (segment (start 153.67 115.53) (end 153.67 120.65) (width 1.5) (layer F.Cu) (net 4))
 (segment (start 129.58001 109.12999) (end 131.5 107.21) (width 1) (layer B.Cu) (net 4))
 (segment (start 125.18501 109.12999) (end 129.58001 109.12999) (width 1) (layer B.Cu) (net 4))
 (segment (start 125.18501 125.82001) (end 125.18501 109.12999) (width 1) (layer B.Cu) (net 4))
 (segment (start 131.5 107.21) (end 131.5 106.91) (width 1) (layer B.Cu) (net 4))
 (segment (start 125.18501 109.12999) (end 125.18501 98.96999) (width 1) (layer B.Cu) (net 4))
 (segment (start 128.5 115.34) (end 128.215 115.34) (width 1) (layer B.Cu) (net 4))
 (segment (start 129.58001 114.25999) (end 128.5 115.34) (width 1) (layer B.Cu) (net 4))
 (segment (start 129.58001 109.12999) (end 129.58001 114.25999) (width 1) (layer B.Cu) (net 4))
 (segment (start 153.67 110.73) (end 154.545 109.855) (width 1.5) (layer B.Cu) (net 6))
 (segment (start 153.67 113.03) (end 153.67 110.73) (width 1.5) (layer B.Cu) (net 6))
 (segment (start 154.545 109.855) (end 167.005 109.855) (width 1.5) (layer B.Cu) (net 6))
 (segment (start 167.64 109.22) (end 167.64 106.68) (width 1.5) (layer B.Cu) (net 6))
 (segment (start 167.005 109.855) (end 167.64 109.22) (width 1.5) (layer B.Cu) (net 6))
 (segment (start 162.56 115.49) (end 165.02 113.03) (width 1.5) (layer B.Cu) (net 8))
 (segment (start 162.56 121.92) (end 162.56 115.49) (width 1.5) (layer B.Cu) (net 8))
 (segment (start 171.53 119.3) (end 171.53 115.57) (width 1.5) (layer B.Cu) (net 8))
 (segment (start 168.91 121.92) (end 171.53 119.3) (width 1.5) (layer B.Cu) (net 8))
 (segment (start 162.56 121.92) (end 168.91 121.92) (width 1.5) (layer B.Cu) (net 8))
 (segment (start 150.4 100.33) (end 150.4 97.79) (width 1) (layer B.Cu) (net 8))
 (segment (start 153.035 118.11) (end 150.4 115.475) (width 1) (layer B.Cu) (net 8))
 (segment (start 150.4 115.475) (end 150.4 100.33) (width 1) (layer B.Cu) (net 8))
 (segment (start 158.75 118.11) (end 153.035 118.11) (width 1) (layer B.Cu) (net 8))
 (segment (start 162.56 121.92) (end 158.75 118.11) (width 1) (layer B.Cu) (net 8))
 (segment (start 178.14 105.41) (end 175.895 103.165) (width 1.5) (layer F.Cu) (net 11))
 (segment (start 180.34 105.41) (end 178.14 105.41) (width 1.5) (layer F.Cu) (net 11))
 (segment (start 175.895 103.165) (end 175.895 100.33) (width 1.5) (layer F.Cu) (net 11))
 (segment (start 175.895 100.33) (end 175.26 99.695) (width 1.5) (layer F.Cu) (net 11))
 (segment (start 164.385 99.695) (end 161.925 97.235) (width 1.5) (layer F.Cu) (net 11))
 (segment (start 175.26 99.695) (end 164.385 99.695) (width 1.5) (layer F.Cu) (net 11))
 (segment (start 160.02 104.14) (end 161.925 102.235) (width 1.5) (layer B.Cu) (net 3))
 (segment (start 160.02 106.68) (end 160.02 104.14) (width 1.5) (layer B.Cu) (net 3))
 (segment (start 177.245 97.235) (end 173.355 97.235) (width 1.5) (layer F.Cu) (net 10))
 (segment (start 177.8 99.695) (end 177.8 97.79) (width 1.5) (layer F.Cu) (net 10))
 (segment (start 177.8 97.79) (end 177.245 97.235) (width 1.5) (layer F.Cu) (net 10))
 (segment (start 179.515 101.41) (end 177.8 99.695) (width 1.5) (layer F.Cu) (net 10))
 (segment (start 180.34 101.41) (end 179.515 101.41) (width 1.5) (layer F.Cu) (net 10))
 (segment (start 165.1 106.68) (end 165.1 104.14) (width 1.5) (layer B.Cu) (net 5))
 (segment (start 165.1 104.14) (end 167.005 102.235) (width 1.5) (layer B.Cu) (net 5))
 (segment (start 167.005 102.235) (end 173.355 102.235) (width 1.5) (layer B.Cu) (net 5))
 (segment (start 152.4 95.885) (end 152.4 97.79) (width 0.5) (layer F.Cu) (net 9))
 (segment (start 151.765 95.25) (end 152.4 95.885) (width 0.5) (layer F.Cu) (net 9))
 (segment (start 137.792208 102.235) (end 141.605 102.235) (width 0.5) (layer F.Cu) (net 9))
 (segment (start 141.605 102.235) (end 143.51 100.33) (width 0.5) (layer F.Cu) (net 9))
 (segment (start 137.16 101.602792) (end 137.792208 102.235) (width 0.5) (layer F.Cu) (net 9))
 (segment (start 144.78 95.25) (end 151.765 95.25) (width 0.5) (layer F.Cu) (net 9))
 (segment (start 143.51 100.33) (end 143.51 96.52) (width 0.5) (layer F.Cu) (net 9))
 (segment (start 143.51 96.52) (end 144.78 95.25) (width 0.5) (layer F.Cu) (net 9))
 (segment (start 137.16 100.33) (end 137.16 101.602792) (width 0.5) (layer F.Cu) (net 9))
 (segment (start 139.7 97.155) (end 140.97 95.885) (width 0.5) (layer F.Cu) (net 21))
 (segment (start 139.7 100.33) (end 139.7 97.155) (width 0.5) (layer F.Cu) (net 21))
 (segment (start 148.59 105.64) (end 148.36 105.41) (width 1.5) (layer F.Cu) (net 1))
 (segment (start 148.59 110.49) (end 148.59 105.64) (width 1.5) (layer F.Cu) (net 1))
 (segment (start 151.13 105.41) (end 152.4 106.68) (width 1.5) (layer F.Cu) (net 1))
 (segment (start 148.36 105.41) (end 151.13 105.41) (width 1.5) (layer F.Cu) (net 1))
 (segment (start 148.59 121.92) (end 148.59 116.84) (width 1.5) (layer F.Cu) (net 7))
 (segment (start 148.59 116.84) (end 148.59 114.3) (width 1.5) (layer F.Cu) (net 7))
 (segment (start 148.59 114.3) (end 153.035 109.855) (width 1.5) (layer F.Cu) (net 7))
 (segment (start 153.035 109.855) (end 171.45 109.855) (width 1.5) (layer F.Cu) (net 7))
 (segment (start 171.45 109.855) (end 172.72 108.585) (width 1.5) (layer F.Cu) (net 7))
 (segment (start 172.72 108.585) (end 172.72 106.68) (width 1.5) (layer F.Cu) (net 7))
 (segment (start 148.4 102.58) (end 148.69 102.87) (width 1) (layer F.Cu) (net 2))
 (segment (start 148.4 100.33) (end 148.4 102.58) (width 1) (layer F.Cu) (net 2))
 (segment (start 148.69 102.87) (end 152.4 102.87) (width 1) (layer F.Cu) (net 2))
 (segment (start 154.94 105.41) (end 154.94 106.68) (width 1) (layer F.Cu) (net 2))
 (segment (start 152.4 102.87) (end 154.94 105.41) (width 1) (layer F.Cu) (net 2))
 (segment (start 154.94 106.68) (end 157.48 106.68) (width 1) (layer F.Cu) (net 2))
 (segment (start 148.4 100.33) (end 148.4 97.79) (width 1) (layer F.Cu) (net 2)))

